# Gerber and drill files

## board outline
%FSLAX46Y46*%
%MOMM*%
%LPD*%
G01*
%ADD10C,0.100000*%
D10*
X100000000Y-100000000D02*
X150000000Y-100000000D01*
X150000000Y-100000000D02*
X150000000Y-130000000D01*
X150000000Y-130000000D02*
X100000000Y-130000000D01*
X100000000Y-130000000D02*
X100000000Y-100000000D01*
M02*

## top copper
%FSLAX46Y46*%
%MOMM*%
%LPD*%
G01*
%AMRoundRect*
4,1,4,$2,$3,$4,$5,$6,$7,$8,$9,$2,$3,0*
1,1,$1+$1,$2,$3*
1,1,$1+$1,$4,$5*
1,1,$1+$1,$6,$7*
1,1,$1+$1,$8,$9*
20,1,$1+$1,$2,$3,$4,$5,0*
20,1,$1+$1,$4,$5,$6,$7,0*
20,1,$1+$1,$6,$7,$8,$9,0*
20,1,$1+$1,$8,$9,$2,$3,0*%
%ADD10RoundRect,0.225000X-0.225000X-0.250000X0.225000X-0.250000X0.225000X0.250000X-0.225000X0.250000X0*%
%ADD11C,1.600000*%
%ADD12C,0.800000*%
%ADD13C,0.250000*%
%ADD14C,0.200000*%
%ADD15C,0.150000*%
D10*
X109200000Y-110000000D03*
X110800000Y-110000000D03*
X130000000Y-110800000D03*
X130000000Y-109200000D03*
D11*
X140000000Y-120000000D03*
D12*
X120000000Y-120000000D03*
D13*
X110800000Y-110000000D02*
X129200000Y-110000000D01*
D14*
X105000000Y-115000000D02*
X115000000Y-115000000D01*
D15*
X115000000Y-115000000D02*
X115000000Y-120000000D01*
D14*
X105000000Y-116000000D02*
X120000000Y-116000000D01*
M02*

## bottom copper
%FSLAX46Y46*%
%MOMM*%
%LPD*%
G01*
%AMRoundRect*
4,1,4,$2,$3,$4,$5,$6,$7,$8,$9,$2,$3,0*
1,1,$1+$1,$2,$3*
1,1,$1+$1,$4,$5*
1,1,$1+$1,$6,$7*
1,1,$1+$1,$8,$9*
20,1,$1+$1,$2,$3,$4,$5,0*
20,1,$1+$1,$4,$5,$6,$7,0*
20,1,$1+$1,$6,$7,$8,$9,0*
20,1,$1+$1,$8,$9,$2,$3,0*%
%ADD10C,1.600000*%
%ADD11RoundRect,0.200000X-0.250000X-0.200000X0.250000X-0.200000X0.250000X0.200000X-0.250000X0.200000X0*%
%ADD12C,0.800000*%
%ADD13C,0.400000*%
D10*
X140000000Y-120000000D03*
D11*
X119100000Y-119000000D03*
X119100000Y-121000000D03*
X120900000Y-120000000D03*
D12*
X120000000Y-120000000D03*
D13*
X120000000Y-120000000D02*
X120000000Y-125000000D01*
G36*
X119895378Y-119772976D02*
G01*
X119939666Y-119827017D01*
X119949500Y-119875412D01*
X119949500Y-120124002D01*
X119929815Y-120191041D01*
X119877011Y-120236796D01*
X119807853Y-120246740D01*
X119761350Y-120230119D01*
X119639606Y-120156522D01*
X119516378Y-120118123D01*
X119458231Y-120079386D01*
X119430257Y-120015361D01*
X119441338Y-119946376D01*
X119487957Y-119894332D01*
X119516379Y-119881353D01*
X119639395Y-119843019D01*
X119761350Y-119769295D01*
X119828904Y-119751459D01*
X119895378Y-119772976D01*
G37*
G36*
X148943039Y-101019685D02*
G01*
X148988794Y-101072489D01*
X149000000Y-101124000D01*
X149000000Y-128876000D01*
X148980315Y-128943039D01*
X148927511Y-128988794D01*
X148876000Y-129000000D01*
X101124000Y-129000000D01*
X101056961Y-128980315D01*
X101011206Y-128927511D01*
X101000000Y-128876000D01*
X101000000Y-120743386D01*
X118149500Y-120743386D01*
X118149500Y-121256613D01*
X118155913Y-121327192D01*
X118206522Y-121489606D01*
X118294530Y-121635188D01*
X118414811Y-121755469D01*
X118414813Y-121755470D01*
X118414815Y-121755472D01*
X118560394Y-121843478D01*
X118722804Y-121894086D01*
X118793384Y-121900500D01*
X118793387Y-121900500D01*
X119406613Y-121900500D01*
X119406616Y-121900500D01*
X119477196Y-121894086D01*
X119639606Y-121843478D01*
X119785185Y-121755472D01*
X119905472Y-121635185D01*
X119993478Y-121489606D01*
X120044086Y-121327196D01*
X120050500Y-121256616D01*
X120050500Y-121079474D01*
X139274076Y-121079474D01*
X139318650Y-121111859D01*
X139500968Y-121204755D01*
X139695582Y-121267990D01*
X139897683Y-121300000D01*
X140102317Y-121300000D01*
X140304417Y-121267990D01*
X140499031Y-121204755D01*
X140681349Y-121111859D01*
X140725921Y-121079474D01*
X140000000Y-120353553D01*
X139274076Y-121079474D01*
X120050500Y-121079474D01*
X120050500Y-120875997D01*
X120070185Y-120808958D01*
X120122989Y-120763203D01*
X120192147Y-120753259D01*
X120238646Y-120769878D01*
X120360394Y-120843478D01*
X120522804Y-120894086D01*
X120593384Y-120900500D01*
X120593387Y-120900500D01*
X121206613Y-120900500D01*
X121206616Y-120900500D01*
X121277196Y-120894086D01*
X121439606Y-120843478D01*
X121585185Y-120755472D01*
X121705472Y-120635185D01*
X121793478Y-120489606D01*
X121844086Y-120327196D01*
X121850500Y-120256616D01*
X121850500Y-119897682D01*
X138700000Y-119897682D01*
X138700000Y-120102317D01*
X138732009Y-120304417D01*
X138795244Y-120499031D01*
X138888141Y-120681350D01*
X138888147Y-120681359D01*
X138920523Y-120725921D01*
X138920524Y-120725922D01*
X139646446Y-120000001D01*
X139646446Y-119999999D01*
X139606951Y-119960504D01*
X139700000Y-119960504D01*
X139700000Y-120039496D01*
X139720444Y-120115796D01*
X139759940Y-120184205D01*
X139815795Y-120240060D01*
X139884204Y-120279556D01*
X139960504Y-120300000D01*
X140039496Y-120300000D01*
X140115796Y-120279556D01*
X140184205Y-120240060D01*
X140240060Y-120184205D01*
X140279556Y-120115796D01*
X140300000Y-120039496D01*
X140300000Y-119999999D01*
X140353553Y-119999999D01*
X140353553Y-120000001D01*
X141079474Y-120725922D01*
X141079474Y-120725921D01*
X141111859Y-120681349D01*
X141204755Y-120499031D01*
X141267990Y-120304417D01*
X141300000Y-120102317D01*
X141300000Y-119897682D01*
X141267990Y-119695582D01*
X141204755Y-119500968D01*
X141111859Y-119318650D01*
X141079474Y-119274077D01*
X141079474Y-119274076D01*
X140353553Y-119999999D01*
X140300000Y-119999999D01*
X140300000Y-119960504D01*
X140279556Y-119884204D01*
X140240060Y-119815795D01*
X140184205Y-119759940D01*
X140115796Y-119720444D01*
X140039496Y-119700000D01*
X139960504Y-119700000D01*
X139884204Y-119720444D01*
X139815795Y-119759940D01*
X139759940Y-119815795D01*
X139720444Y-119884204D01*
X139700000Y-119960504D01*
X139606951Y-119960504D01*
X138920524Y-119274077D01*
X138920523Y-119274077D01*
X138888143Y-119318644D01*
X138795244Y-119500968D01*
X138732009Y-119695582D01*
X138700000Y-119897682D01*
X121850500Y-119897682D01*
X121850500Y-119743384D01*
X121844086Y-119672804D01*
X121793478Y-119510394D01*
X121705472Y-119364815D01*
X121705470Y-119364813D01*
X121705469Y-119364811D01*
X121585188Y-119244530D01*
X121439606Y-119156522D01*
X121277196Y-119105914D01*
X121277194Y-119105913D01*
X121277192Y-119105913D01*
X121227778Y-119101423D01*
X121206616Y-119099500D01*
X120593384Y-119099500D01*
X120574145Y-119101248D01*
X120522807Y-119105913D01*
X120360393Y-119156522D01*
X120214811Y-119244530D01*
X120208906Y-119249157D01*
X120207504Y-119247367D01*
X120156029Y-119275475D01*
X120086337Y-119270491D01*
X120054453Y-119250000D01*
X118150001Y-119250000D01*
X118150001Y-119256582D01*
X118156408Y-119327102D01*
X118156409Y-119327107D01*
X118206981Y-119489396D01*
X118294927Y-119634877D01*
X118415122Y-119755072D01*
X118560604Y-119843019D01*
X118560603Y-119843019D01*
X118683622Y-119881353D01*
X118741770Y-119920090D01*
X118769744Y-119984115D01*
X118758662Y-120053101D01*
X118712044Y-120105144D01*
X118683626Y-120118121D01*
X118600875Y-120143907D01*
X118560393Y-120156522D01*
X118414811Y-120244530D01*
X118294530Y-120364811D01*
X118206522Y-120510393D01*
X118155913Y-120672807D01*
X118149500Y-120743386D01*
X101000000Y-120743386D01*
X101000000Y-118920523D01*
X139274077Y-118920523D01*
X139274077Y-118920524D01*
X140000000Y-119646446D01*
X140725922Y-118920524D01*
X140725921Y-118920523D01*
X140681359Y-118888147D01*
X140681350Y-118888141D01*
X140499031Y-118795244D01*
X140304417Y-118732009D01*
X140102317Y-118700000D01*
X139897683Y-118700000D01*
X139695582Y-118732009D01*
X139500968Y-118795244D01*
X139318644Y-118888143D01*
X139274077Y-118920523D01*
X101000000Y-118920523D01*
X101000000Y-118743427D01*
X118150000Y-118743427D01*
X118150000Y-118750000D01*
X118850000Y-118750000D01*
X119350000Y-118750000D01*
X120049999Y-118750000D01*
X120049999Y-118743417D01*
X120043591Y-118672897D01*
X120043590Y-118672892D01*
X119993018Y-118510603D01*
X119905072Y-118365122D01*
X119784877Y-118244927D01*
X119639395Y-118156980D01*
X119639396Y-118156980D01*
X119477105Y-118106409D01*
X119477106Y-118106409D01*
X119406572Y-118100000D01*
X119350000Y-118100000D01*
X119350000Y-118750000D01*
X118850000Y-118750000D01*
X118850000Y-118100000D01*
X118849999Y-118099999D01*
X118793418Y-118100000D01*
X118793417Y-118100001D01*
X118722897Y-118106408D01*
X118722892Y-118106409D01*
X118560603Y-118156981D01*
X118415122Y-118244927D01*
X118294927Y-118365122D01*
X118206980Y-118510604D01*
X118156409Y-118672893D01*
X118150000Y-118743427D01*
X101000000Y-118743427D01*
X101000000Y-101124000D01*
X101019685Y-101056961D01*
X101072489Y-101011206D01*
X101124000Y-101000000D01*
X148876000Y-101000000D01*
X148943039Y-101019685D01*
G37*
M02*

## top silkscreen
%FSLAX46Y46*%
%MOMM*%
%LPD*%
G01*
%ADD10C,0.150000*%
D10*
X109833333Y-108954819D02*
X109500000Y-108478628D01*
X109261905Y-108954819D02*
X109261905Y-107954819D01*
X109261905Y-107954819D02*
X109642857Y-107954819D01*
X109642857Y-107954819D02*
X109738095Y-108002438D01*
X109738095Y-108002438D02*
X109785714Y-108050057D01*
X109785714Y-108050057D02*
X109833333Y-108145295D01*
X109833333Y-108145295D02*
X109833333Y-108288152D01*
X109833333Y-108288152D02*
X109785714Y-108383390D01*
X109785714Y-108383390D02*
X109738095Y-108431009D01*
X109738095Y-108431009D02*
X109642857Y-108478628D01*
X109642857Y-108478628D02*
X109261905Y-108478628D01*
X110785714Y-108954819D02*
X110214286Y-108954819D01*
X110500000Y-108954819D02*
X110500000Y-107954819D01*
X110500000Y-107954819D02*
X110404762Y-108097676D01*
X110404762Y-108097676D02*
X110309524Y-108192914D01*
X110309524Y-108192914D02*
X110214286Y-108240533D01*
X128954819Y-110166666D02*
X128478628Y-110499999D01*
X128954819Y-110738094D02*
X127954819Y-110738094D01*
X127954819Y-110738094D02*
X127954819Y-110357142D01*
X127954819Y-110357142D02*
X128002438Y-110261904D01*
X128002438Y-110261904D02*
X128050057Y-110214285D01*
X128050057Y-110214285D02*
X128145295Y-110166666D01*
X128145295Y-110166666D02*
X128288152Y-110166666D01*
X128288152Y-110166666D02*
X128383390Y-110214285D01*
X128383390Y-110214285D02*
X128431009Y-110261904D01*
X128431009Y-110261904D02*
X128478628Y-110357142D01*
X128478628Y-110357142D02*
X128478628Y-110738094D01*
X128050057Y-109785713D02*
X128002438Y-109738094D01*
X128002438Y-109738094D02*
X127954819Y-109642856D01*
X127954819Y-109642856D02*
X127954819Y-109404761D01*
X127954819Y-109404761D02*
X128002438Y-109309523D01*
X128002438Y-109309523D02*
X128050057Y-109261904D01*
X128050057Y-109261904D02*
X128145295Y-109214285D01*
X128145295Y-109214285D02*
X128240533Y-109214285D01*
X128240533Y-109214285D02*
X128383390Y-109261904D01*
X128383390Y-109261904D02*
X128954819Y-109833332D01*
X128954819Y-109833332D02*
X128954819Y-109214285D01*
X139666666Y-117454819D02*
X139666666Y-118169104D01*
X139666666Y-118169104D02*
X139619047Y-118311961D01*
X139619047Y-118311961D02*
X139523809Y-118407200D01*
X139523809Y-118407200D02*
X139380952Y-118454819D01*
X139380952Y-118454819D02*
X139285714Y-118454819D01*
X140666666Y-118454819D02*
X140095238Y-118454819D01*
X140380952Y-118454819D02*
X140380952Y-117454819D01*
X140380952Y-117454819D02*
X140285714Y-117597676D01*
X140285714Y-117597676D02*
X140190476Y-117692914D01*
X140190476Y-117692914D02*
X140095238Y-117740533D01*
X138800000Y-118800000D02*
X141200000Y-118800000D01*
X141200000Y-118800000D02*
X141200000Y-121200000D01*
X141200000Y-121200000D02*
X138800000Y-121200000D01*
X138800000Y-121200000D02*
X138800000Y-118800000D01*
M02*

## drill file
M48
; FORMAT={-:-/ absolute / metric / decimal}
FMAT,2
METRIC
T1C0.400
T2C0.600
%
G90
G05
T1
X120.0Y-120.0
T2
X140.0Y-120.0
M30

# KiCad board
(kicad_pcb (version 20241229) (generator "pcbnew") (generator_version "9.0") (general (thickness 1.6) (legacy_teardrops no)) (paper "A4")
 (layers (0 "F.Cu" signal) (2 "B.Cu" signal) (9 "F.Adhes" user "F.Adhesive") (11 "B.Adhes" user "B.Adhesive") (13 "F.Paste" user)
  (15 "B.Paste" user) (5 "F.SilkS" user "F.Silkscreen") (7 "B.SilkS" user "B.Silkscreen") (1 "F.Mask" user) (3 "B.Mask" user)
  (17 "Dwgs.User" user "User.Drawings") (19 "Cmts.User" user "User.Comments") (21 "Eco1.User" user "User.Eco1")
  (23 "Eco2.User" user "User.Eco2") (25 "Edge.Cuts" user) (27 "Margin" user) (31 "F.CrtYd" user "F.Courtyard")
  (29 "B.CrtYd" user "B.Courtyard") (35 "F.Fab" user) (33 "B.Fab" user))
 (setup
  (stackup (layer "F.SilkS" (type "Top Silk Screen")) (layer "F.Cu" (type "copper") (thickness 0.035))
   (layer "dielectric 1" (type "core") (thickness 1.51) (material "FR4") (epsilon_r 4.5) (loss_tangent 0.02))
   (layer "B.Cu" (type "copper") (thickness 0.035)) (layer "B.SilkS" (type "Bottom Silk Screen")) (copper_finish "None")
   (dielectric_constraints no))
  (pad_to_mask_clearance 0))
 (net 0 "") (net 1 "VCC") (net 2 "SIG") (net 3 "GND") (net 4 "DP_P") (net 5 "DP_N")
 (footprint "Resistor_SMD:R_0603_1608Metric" (layer "F.Cu") (at 110 110 0)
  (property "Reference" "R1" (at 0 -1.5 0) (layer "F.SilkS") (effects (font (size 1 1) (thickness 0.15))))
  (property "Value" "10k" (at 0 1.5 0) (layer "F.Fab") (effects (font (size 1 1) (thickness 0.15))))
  (pad "1" smd roundrect (at -0.8 0) (size 0.9 0.95) (layers "F.Cu" "F.Paste" "F.Mask") (roundrect_rratio 0.25) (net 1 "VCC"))
  (pad "2" smd roundrect (at 0.8 0) (size 0.9 0.95) (layers "F.Cu" "F.Paste" "F.Mask") (roundrect_rratio 0.25) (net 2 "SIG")))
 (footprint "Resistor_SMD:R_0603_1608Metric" (layer "F.Cu") (at 130 110 90)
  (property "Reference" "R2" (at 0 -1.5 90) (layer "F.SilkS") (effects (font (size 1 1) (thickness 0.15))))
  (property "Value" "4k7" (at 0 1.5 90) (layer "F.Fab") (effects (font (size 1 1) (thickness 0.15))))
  (pad "1" smd roundrect (at -0.8 0) (size 0.9 0.95) (layers "F.Cu" "F.Paste" "F.Mask") (roundrect_rratio 0.25) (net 2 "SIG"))
  (pad "2" smd roundrect (at 0.8 0) (size 0.9 0.95) (layers "F.Cu" "F.Paste" "F.Mask") (roundrect_rratio 0.25) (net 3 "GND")))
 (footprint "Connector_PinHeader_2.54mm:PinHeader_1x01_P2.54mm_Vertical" (layer "F.Cu") (at 140 120 0)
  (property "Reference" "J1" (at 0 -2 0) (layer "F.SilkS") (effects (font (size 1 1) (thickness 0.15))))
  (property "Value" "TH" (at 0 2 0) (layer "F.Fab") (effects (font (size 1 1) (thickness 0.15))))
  (fp_line (start -1.2 -1.2) (end 1.2 -1.2) (stroke (width 0.15) (type solid)) (layer "F.SilkS"))
  (fp_line (start 1.2 -1.2) (end 1.2 1.2) (stroke (width 0.15) (type solid)) (layer "F.SilkS"))
  (fp_line (start 1.2 1.2) (end -1.2 1.2) (stroke (width 0.15) (type solid)) (layer "F.SilkS"))
  (fp_line (start -1.2 1.2) (end -1.2 -1.2) (stroke (width 0.15) (type solid)) (layer "F.SilkS"))
  (pad "1" thru_hole circle (at 0 0) (size 1.6 1.6) (drill 0.6) (layers "*.Cu" "*.Mask") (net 3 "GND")))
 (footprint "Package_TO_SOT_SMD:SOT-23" (layer "B.Cu") (at 120 120 0)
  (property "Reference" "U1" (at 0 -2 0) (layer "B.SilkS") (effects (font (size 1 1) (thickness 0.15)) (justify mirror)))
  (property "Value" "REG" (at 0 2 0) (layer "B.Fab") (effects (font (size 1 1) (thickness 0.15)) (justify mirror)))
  (pad "1" smd roundrect (at -0.9 -1) (size 0.9 0.8) (layers "B.Cu" "B.Paste" "B.Mask") (roundrect_rratio 0.25) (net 3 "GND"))
  (pad "2" smd roundrect (at -0.9 1) (size 0.9 0.8) (layers "B.Cu" "B.Paste" "B.Mask") (roundrect_rratio 0.25) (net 1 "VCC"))
  (pad "3" smd roundrect (at 0.9 0) (size 0.9 0.8) (layers "B.Cu" "B.Paste" "B.Mask") (roundrect_rratio 0.25) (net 2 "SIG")))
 (gr_line (start 100 100) (end 150 100) (stroke (width 0.1) (type solid)) (layer "Edge.Cuts"))
 (gr_line (start 150 100) (end 150 130) (stroke (width 0.1) (type solid)) (layer "Edge.Cuts"))
 (gr_line (start 150 130) (end 100 130) (stroke (width 0.1) (type solid)) (layer "Edge.Cuts"))
 (gr_line (start 100 130) (end 100 100) (stroke (width 0.1) (type solid)) (layer "Edge.Cuts"))
 (segment (start 110.8 110) (end 129.2 110) (width 0.25) (layer "F.Cu") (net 2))
 (segment (start 120 120) (end 120 125) (width 0.4) (layer "B.Cu") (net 3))
 (via (at 120 120) (size 0.8) (drill 0.4) (layers "F.Cu" "B.Cu") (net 3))
 (segment (start 105 115) (end 115 115) (width 0.2) (layer "F.Cu") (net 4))
 (segment (start 115 115) (end 115 120) (width 0.15) (layer "F.Cu") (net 4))
 (segment (start 105 116) (end 120 116) (width 0.2) (layer "F.Cu") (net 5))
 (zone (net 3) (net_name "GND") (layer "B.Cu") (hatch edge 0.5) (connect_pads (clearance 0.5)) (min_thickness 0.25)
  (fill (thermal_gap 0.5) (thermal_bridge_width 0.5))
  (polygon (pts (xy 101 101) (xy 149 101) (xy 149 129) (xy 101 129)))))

